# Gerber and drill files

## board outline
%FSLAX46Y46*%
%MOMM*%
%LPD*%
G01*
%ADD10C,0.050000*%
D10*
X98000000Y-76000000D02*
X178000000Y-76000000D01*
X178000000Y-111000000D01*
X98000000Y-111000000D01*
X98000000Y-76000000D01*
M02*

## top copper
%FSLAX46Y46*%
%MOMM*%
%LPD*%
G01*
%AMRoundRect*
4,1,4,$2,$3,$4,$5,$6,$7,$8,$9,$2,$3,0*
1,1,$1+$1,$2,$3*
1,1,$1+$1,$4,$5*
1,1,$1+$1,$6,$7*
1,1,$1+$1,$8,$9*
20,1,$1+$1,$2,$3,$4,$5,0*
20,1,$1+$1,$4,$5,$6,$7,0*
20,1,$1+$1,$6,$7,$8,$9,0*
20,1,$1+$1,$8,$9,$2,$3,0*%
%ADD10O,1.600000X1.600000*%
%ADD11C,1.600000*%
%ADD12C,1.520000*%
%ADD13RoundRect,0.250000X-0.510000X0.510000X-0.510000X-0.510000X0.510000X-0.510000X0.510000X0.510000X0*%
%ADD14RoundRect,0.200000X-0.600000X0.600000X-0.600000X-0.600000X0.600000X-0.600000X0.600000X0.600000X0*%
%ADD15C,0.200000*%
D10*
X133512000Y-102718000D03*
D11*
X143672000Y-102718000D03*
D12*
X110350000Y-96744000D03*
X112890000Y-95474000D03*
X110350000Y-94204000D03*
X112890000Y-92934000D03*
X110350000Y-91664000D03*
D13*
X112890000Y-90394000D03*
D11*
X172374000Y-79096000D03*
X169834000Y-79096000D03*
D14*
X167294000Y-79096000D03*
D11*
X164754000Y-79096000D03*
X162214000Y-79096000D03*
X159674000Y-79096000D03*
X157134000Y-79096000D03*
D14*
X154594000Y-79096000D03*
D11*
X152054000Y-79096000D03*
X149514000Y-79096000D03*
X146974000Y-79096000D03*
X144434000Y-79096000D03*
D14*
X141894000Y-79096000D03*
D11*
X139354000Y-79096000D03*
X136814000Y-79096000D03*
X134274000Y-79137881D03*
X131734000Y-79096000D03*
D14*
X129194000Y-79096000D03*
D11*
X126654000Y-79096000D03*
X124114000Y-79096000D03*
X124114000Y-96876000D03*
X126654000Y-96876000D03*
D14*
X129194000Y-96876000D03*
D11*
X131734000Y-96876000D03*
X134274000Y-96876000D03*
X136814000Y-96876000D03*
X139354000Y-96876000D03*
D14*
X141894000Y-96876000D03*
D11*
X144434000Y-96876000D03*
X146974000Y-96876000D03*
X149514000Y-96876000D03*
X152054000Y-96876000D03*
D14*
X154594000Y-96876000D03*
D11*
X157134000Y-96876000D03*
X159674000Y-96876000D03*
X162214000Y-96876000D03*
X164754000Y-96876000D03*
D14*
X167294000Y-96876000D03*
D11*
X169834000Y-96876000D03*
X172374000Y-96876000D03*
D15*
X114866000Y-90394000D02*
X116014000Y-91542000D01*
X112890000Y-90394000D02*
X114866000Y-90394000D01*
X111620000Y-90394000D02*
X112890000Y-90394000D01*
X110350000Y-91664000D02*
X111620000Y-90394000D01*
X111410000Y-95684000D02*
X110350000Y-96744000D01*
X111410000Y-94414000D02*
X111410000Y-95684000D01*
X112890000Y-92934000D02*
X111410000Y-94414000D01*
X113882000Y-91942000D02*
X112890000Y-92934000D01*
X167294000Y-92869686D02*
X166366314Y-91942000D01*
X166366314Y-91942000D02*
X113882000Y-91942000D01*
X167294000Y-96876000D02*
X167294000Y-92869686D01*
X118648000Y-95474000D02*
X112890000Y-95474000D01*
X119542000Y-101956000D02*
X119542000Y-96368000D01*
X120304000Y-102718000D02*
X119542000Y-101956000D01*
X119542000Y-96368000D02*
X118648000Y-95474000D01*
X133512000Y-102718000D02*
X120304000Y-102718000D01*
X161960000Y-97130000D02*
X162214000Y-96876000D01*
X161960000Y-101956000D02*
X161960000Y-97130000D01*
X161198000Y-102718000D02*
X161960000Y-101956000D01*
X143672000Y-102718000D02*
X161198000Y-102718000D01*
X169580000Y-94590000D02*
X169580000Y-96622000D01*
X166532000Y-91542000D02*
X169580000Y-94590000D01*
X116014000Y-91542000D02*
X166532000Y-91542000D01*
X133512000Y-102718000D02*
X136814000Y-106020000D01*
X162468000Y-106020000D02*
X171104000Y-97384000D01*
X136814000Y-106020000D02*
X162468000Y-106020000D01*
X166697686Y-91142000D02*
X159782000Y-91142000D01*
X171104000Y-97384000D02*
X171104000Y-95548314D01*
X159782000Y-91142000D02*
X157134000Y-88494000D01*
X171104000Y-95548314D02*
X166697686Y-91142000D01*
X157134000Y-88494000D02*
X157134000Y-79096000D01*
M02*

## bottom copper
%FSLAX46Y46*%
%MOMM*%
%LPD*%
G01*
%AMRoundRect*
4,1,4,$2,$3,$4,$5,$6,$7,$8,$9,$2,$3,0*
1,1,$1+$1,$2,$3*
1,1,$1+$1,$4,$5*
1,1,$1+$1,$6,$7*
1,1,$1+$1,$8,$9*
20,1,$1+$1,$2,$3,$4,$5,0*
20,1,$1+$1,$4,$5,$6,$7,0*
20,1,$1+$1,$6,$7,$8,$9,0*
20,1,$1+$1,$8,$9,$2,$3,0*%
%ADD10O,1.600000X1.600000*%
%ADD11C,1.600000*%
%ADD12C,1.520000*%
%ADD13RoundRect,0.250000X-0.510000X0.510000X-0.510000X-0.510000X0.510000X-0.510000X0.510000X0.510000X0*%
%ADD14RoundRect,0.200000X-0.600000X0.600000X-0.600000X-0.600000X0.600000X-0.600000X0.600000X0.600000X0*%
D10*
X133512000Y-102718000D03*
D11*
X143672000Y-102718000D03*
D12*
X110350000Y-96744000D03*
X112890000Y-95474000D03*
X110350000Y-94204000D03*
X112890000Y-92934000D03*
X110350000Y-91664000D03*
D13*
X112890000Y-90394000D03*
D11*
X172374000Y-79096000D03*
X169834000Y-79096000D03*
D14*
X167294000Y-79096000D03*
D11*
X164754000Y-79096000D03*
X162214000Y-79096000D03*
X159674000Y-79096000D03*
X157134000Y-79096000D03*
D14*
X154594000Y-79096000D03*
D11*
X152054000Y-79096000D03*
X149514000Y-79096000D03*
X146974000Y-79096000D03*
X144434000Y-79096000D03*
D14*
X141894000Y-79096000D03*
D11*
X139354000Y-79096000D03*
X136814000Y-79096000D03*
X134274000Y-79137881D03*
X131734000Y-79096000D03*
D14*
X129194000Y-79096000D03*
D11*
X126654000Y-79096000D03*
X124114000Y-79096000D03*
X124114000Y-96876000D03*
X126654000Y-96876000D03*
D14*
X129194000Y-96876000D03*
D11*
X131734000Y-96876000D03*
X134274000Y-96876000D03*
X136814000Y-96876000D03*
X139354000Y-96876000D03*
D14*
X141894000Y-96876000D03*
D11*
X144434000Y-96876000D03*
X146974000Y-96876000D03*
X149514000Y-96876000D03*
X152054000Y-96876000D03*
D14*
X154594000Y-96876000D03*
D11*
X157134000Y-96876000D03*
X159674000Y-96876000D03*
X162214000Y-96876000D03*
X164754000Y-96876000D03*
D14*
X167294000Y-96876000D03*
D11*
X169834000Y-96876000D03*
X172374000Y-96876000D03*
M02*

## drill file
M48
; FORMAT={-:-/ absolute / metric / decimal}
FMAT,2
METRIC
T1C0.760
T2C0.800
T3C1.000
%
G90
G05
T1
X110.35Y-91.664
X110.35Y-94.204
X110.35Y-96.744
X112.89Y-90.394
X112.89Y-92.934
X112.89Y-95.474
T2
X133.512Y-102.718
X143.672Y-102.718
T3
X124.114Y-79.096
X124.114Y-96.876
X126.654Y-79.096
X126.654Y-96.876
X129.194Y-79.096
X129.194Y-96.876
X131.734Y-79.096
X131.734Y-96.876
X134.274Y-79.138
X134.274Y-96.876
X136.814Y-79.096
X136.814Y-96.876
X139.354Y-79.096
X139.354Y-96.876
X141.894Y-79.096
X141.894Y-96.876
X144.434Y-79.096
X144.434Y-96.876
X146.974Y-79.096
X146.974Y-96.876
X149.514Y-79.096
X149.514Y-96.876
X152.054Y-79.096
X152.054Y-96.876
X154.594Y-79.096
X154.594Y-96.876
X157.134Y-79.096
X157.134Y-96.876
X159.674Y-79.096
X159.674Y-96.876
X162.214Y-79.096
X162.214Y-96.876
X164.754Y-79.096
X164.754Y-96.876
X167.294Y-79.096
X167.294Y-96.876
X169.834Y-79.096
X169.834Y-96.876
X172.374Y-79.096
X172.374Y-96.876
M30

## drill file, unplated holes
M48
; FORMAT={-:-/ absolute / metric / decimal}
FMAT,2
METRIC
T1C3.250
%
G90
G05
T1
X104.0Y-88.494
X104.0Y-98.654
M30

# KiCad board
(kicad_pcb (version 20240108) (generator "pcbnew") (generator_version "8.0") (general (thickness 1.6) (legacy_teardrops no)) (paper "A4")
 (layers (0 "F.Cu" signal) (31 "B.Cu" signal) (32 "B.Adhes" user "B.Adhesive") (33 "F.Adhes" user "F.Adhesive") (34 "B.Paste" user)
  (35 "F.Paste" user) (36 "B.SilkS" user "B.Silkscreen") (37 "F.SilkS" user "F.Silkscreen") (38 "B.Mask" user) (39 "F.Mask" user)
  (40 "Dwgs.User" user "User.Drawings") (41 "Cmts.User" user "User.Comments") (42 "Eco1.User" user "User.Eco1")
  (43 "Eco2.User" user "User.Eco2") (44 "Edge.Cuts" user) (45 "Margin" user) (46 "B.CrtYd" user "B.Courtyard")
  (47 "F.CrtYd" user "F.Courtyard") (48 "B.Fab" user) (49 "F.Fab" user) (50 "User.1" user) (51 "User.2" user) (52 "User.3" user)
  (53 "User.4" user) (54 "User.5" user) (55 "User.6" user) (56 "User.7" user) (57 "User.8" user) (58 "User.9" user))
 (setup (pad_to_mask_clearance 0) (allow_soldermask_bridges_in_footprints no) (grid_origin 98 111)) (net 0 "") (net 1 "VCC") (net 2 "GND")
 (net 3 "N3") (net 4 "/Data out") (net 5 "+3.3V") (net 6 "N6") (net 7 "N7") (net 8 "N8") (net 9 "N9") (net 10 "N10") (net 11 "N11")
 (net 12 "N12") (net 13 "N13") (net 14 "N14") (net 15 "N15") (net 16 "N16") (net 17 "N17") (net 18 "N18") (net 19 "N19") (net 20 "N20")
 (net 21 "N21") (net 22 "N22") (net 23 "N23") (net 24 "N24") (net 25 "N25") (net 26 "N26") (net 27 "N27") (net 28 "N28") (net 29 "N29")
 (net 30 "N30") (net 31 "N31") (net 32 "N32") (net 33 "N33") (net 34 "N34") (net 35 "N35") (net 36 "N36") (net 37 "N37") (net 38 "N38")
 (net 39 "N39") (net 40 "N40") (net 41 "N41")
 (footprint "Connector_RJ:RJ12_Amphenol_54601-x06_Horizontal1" (layer "F.Cu") (at 112.89 90.394 -90)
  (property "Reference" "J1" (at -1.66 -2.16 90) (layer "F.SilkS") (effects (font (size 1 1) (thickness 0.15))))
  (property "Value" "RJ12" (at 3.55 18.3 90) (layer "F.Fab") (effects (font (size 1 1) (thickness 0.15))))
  (pad "" np_thru_hole circle (at -1.9 8.89 270) (size 3.25 3.25) (drill 3.25) (layers "*.Cu" "*.Mask"))
  (pad "" np_thru_hole circle (at 8.26 8.89 270) (size 3.25 3.25) (drill 3.25) (layers "*.Cu" "*.Mask"))
  (pad "1" thru_hole roundrect (at 0 0 270) (size 1.52 1.52) (drill 0.76) (layers "*.Cu" "*.Mask") (remove_unused_layers no)
   (roundrect_rratio 0.1644736842) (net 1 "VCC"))
  (pad "2" thru_hole circle (at 1.27 2.54 270) (size 1.52 1.52) (drill 0.76) (layers "*.Cu" "*.Mask") (remove_unused_layers no)
   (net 1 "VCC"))
  (pad "3" thru_hole circle (at 2.54 0 270) (size 1.52 1.52) (drill 0.76) (layers "*.Cu" "*.Mask") (remove_unused_layers no) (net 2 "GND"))
  (pad "4" thru_hole circle (at 3.81 2.54 270) (size 1.52 1.52) (drill 0.76) (layers "*.Cu" "*.Mask") (remove_unused_layers no) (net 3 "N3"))
  (pad "5" thru_hole circle (at 5.08 0 270) (size 1.52 1.52) (drill 0.76) (layers "*.Cu" "*.Mask") (remove_unused_layers no)
   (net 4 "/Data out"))
  (pad "6" thru_hole circle (at 6.35 2.54 270) (size 1.52 1.52) (drill 0.76) (layers "*.Cu" "*.Mask") (remove_unused_layers no)
   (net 2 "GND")))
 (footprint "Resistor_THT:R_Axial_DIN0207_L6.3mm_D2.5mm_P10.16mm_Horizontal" (layer "F.Cu") (at 143.672 102.718 180)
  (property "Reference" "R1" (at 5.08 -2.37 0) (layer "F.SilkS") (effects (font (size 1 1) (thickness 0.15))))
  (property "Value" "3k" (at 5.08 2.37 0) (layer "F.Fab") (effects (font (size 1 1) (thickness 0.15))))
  (pad "1" thru_hole circle (at 0 0 180) (size 1.6 1.6) (drill 0.8) (layers "*.Cu" "*.Mask") (remove_unused_layers no) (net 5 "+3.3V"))
  (pad "2" thru_hole oval (at 10.16 0 180) (size 1.6 1.6) (drill 0.8) (layers "*.Cu" "*.Mask") (remove_unused_layers no) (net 4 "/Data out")))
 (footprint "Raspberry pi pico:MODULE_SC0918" (layer "F.Cu") (at 148.244 87.986 -90)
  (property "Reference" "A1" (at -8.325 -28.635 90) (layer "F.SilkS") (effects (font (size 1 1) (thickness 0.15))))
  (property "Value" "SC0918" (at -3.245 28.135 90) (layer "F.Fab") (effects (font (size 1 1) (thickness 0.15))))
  (pad "1" thru_hole circle (at -8.89 -24.13 270) (size 1.6 1.6) (drill 1) (layers "*.Cu" "*.Mask") (remove_unused_layers no) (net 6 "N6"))
  (pad "2" thru_hole circle (at -8.89 -21.59 270) (size 1.6 1.6) (drill 1) (layers "*.Cu" "*.Mask") (remove_unused_layers no) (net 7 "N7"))
  (pad "3" thru_hole roundrect (at -8.89 -19.05 270) (size 1.6 1.6) (drill 1) (layers "*.Cu" "*.Mask") (remove_unused_layers no)
   (roundrect_rratio 0.125) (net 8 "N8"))
  (pad "4" thru_hole circle (at -8.89 -16.51 270) (size 1.6 1.6) (drill 1) (layers "*.Cu" "*.Mask") (remove_unused_layers no) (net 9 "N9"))
  (pad "5" thru_hole circle (at -8.89 -13.97 270) (size 1.6 1.6) (drill 1) (layers "*.Cu" "*.Mask") (remove_unused_layers no) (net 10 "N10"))
  (pad "6" thru_hole circle (at -8.89 -11.43 270) (size 1.6 1.6) (drill 1) (layers "*.Cu" "*.Mask") (remove_unused_layers no) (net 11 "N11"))
  (pad "7" thru_hole circle (at -8.89 -8.89 270) (size 1.6 1.6) (drill 1) (layers "*.Cu" "*.Mask") (remove_unused_layers no)
   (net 4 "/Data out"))
  (pad "8" thru_hole roundrect (at -8.89 -6.35 270) (size 1.6 1.6) (drill 1) (layers "*.Cu" "*.Mask") (remove_unused_layers no)
   (roundrect_rratio 0.125) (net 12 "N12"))
  (pad "9" thru_hole circle (at -8.89 -3.81 270) (size 1.6 1.6) (drill 1) (layers "*.Cu" "*.Mask") (remove_unused_layers no) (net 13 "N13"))
  (pad "10" thru_hole circle (at -8.89 -1.27 270) (size 1.6 1.6) (drill 1) (layers "*.Cu" "*.Mask") (remove_unused_layers no) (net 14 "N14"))
  (pad "11" thru_hole circle (at -8.89 1.27 270) (size 1.6 1.6) (drill 1) (layers "*.Cu" "*.Mask") (remove_unused_layers no) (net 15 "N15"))
  (pad "12" thru_hole circle (at -8.89 3.81 270) (size 1.6 1.6) (drill 1) (layers "*.Cu" "*.Mask") (remove_unused_layers no) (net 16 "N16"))
  (pad "13" thru_hole roundrect (at -8.89 6.35 270) (size 1.6 1.6) (drill 1) (layers "*.Cu" "*.Mask") (remove_unused_layers no)
   (roundrect_rratio 0.125) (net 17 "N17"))
  (pad "14" thru_hole circle (at -8.89 8.89 270) (size 1.6 1.6) (drill 1) (layers "*.Cu" "*.Mask") (remove_unused_layers no) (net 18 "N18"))
  (pad "15" thru_hole circle (at -8.89 11.43 270) (size 1.6 1.6) (drill 1) (layers "*.Cu" "*.Mask") (remove_unused_layers no) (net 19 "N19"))
  (pad "16" thru_hole circle (at -8.848119 13.97 270) (size 1.6 1.6) (drill 1) (layers "*.Cu" "*.Mask") (remove_unused_layers no)
   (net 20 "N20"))
  (pad "17" thru_hole circle (at -8.89 16.51 270) (size 1.6 1.6) (drill 1) (layers "*.Cu" "*.Mask") (remove_unused_layers no) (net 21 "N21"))
  (pad "18" thru_hole roundrect (at -8.89 19.05 270) (size 1.6 1.6) (drill 1) (layers "*.Cu" "*.Mask") (remove_unused_layers no)
   (roundrect_rratio 0.125) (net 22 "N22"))
  (pad "19" thru_hole circle (at -8.89 21.59 270) (size 1.6 1.6) (drill 1) (layers "*.Cu" "*.Mask") (remove_unused_layers no) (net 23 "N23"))
  (pad "20" thru_hole circle (at -8.89 24.13 270) (size 1.6 1.6) (drill 1) (layers "*.Cu" "*.Mask") (remove_unused_layers no) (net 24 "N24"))
  (pad "21" thru_hole circle (at 8.89 24.13 270) (size 1.6 1.6) (drill 1) (layers "*.Cu" "*.Mask") (remove_unused_layers no) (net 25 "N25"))
  (pad "22" thru_hole circle (at 8.89 21.59 270) (size 1.6 1.6) (drill 1) (layers "*.Cu" "*.Mask") (remove_unused_layers no) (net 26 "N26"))
  (pad "23" thru_hole roundrect (at 8.89 19.05 270) (size 1.6 1.6) (drill 1) (layers "*.Cu" "*.Mask") (remove_unused_layers no)
   (roundrect_rratio 0.125) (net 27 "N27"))
  (pad "24" thru_hole circle (at 8.89 16.51 270) (size 1.6 1.6) (drill 1) (layers "*.Cu" "*.Mask") (remove_unused_layers no) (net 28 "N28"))
  (pad "25" thru_hole circle (at 8.89 13.97 270) (size 1.6 1.6) (drill 1) (layers "*.Cu" "*.Mask") (remove_unused_layers no) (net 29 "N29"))
  (pad "26" thru_hole circle (at 8.89 11.43 270) (size 1.6 1.6) (drill 1) (layers "*.Cu" "*.Mask") (remove_unused_layers no) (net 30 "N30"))
  (pad "27" thru_hole circle (at 8.89 8.89 270) (size 1.6 1.6) (drill 1) (layers "*.Cu" "*.Mask") (remove_unused_layers no) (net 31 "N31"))
  (pad "28" thru_hole roundrect (at 8.89 6.35 270) (size 1.6 1.6) (drill 1) (layers "*.Cu" "*.Mask") (remove_unused_layers no)
   (roundrect_rratio 0.125) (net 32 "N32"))
  (pad "29" thru_hole circle (at 8.89 3.81 270) (size 1.6 1.6) (drill 1) (layers "*.Cu" "*.Mask") (remove_unused_layers no) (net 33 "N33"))
  (pad "30" thru_hole circle (at 8.89 1.27 270) (size 1.6 1.6) (drill 1) (layers "*.Cu" "*.Mask") (remove_unused_layers no) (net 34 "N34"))
  (pad "31" thru_hole circle (at 8.89 -1.27 270) (size 1.6 1.6) (drill 1) (layers "*.Cu" "*.Mask") (remove_unused_layers no) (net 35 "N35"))
  (pad "32" thru_hole circle (at 8.89 -3.81 270) (size 1.6 1.6) (drill 1) (layers "*.Cu" "*.Mask") (remove_unused_layers no) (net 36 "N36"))
  (pad "33" thru_hole roundrect (at 8.89 -6.35 270) (size 1.6 1.6) (drill 1) (layers "*.Cu" "*.Mask") (remove_unused_layers no)
   (roundrect_rratio 0.125) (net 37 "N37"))
  (pad "34" thru_hole circle (at 8.89 -8.89 270) (size 1.6 1.6) (drill 1) (layers "*.Cu" "*.Mask") (remove_unused_layers no) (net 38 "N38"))
  (pad "35" thru_hole circle (at 8.89 -11.43 270) (size 1.6 1.6) (drill 1) (layers "*.Cu" "*.Mask") (remove_unused_layers no) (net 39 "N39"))
  (pad "36" thru_hole circle (at 8.89 -13.97 270) (size 1.6 1.6) (drill 1) (layers "*.Cu" "*.Mask") (remove_unused_layers no)
   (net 5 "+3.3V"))
  (pad "37" thru_hole circle (at 8.89 -16.51 270) (size 1.6 1.6) (drill 1) (layers "*.Cu" "*.Mask") (remove_unused_layers no) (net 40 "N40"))
  (pad "38" thru_hole roundrect (at 8.89 -19.05 270) (size 1.6 1.6) (drill 1) (layers "*.Cu" "*.Mask") (remove_unused_layers no)
   (roundrect_rratio 0.125) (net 2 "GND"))
  (pad "39" thru_hole circle (at 8.89 -21.59 270) (size 1.6 1.6) (drill 1) (layers "*.Cu" "*.Mask") (remove_unused_layers no) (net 1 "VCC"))
  (pad "40" thru_hole circle (at 8.89 -24.13 270) (size 1.6 1.6) (drill 1) (layers "*.Cu" "*.Mask") (remove_unused_layers no) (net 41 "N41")))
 (gr_rect (start 98 76) (end 178 111) (stroke (width 0.05) (type default)) (fill none) (layer "Edge.Cuts"))
 (segment (start 143.672 102.718) (end 161.198 102.718) (width 0.2) (layer "F.Cu") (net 5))
 (segment (start 161.96 101.956) (end 161.96 97.13) (width 0.2) (layer "F.Cu") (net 5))
 (segment (start 161.198 102.718) (end 161.96 101.956) (width 0.2) (layer "F.Cu") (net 5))
 (segment (start 161.96 97.13) (end 162.214 96.876) (width 0.2) (layer "F.Cu") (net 5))
 (segment (start 119.542 101.956) (end 119.542 96.368) (width 0.2) (layer "F.Cu") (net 4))
 (segment (start 162.468 106.02) (end 171.104 97.384) (width 0.2) (layer "F.Cu") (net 4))
 (segment (start 166.697686 91.142) (end 159.782 91.142) (width 0.2) (layer "F.Cu") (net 4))
 (segment (start 119.542 96.368) (end 118.648 95.474) (width 0.2) (layer "F.Cu") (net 4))
 (segment (start 133.512 102.718) (end 120.304 102.718) (width 0.2) (layer "F.Cu") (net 4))
 (segment (start 171.104 97.384) (end 171.104 95.548314) (width 0.2) (layer "F.Cu") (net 4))
 (segment (start 118.648 95.474) (end 112.89 95.474) (width 0.2) (layer "F.Cu") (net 4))
 (segment (start 171.104 95.548314) (end 166.697686 91.142) (width 0.2) (layer "F.Cu") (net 4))
 (segment (start 136.814 106.02) (end 162.468 106.02) (width 0.2) (layer "F.Cu") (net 4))
 (segment (start 157.134 88.494) (end 157.134 79.096) (width 0.2) (layer "F.Cu") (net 4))
 (segment (start 159.782 91.142) (end 157.134 88.494) (width 0.2) (layer "F.Cu") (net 4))
 (segment (start 120.304 102.718) (end 119.542 101.956) (width 0.2) (layer "F.Cu") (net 4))
 (segment (start 133.512 102.718) (end 136.814 106.02) (width 0.2) (layer "F.Cu") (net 4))
 (segment (start 166.366314 91.942) (end 113.882 91.942) (width 0.2) (layer "F.Cu") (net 2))
 (segment (start 167.294 96.876) (end 167.294 92.869686) (width 0.2) (layer "F.Cu") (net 2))
 (segment (start 111.41 95.684) (end 110.35 96.744) (width 0.2) (layer "F.Cu") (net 2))
 (segment (start 111.41 94.414) (end 111.41 95.684) (width 0.2) (layer "F.Cu") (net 2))
 (segment (start 113.882 91.942) (end 112.89 92.934) (width 0.2) (layer "F.Cu") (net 2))
 (segment (start 167.294 92.869686) (end 166.366314 91.942) (width 0.2) (layer "F.Cu") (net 2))
 (segment (start 112.89 92.934) (end 111.41 94.414) (width 0.2) (layer "F.Cu") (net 2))
 (segment (start 111.62 90.394) (end 112.89 90.394) (width 0.2) (layer "F.Cu") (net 1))
 (segment (start 112.89 90.394) (end 114.866 90.394) (width 0.2) (layer "F.Cu") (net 1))
 (segment (start 169.58 94.59) (end 169.58 96.622) (width 0.2) (layer "F.Cu") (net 1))
 (segment (start 114.866 90.394) (end 116.014 91.542) (width 0.2) (layer "F.Cu") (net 1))
 (segment (start 166.532 91.542) (end 169.58 94.59) (width 0.2) (layer "F.Cu") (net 1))
 (segment (start 116.014 91.542) (end 166.532 91.542) (width 0.2) (layer "F.Cu") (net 1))
 (segment (start 110.35 91.664) (end 111.62 90.394) (width 0.2) (layer "F.Cu") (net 1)))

